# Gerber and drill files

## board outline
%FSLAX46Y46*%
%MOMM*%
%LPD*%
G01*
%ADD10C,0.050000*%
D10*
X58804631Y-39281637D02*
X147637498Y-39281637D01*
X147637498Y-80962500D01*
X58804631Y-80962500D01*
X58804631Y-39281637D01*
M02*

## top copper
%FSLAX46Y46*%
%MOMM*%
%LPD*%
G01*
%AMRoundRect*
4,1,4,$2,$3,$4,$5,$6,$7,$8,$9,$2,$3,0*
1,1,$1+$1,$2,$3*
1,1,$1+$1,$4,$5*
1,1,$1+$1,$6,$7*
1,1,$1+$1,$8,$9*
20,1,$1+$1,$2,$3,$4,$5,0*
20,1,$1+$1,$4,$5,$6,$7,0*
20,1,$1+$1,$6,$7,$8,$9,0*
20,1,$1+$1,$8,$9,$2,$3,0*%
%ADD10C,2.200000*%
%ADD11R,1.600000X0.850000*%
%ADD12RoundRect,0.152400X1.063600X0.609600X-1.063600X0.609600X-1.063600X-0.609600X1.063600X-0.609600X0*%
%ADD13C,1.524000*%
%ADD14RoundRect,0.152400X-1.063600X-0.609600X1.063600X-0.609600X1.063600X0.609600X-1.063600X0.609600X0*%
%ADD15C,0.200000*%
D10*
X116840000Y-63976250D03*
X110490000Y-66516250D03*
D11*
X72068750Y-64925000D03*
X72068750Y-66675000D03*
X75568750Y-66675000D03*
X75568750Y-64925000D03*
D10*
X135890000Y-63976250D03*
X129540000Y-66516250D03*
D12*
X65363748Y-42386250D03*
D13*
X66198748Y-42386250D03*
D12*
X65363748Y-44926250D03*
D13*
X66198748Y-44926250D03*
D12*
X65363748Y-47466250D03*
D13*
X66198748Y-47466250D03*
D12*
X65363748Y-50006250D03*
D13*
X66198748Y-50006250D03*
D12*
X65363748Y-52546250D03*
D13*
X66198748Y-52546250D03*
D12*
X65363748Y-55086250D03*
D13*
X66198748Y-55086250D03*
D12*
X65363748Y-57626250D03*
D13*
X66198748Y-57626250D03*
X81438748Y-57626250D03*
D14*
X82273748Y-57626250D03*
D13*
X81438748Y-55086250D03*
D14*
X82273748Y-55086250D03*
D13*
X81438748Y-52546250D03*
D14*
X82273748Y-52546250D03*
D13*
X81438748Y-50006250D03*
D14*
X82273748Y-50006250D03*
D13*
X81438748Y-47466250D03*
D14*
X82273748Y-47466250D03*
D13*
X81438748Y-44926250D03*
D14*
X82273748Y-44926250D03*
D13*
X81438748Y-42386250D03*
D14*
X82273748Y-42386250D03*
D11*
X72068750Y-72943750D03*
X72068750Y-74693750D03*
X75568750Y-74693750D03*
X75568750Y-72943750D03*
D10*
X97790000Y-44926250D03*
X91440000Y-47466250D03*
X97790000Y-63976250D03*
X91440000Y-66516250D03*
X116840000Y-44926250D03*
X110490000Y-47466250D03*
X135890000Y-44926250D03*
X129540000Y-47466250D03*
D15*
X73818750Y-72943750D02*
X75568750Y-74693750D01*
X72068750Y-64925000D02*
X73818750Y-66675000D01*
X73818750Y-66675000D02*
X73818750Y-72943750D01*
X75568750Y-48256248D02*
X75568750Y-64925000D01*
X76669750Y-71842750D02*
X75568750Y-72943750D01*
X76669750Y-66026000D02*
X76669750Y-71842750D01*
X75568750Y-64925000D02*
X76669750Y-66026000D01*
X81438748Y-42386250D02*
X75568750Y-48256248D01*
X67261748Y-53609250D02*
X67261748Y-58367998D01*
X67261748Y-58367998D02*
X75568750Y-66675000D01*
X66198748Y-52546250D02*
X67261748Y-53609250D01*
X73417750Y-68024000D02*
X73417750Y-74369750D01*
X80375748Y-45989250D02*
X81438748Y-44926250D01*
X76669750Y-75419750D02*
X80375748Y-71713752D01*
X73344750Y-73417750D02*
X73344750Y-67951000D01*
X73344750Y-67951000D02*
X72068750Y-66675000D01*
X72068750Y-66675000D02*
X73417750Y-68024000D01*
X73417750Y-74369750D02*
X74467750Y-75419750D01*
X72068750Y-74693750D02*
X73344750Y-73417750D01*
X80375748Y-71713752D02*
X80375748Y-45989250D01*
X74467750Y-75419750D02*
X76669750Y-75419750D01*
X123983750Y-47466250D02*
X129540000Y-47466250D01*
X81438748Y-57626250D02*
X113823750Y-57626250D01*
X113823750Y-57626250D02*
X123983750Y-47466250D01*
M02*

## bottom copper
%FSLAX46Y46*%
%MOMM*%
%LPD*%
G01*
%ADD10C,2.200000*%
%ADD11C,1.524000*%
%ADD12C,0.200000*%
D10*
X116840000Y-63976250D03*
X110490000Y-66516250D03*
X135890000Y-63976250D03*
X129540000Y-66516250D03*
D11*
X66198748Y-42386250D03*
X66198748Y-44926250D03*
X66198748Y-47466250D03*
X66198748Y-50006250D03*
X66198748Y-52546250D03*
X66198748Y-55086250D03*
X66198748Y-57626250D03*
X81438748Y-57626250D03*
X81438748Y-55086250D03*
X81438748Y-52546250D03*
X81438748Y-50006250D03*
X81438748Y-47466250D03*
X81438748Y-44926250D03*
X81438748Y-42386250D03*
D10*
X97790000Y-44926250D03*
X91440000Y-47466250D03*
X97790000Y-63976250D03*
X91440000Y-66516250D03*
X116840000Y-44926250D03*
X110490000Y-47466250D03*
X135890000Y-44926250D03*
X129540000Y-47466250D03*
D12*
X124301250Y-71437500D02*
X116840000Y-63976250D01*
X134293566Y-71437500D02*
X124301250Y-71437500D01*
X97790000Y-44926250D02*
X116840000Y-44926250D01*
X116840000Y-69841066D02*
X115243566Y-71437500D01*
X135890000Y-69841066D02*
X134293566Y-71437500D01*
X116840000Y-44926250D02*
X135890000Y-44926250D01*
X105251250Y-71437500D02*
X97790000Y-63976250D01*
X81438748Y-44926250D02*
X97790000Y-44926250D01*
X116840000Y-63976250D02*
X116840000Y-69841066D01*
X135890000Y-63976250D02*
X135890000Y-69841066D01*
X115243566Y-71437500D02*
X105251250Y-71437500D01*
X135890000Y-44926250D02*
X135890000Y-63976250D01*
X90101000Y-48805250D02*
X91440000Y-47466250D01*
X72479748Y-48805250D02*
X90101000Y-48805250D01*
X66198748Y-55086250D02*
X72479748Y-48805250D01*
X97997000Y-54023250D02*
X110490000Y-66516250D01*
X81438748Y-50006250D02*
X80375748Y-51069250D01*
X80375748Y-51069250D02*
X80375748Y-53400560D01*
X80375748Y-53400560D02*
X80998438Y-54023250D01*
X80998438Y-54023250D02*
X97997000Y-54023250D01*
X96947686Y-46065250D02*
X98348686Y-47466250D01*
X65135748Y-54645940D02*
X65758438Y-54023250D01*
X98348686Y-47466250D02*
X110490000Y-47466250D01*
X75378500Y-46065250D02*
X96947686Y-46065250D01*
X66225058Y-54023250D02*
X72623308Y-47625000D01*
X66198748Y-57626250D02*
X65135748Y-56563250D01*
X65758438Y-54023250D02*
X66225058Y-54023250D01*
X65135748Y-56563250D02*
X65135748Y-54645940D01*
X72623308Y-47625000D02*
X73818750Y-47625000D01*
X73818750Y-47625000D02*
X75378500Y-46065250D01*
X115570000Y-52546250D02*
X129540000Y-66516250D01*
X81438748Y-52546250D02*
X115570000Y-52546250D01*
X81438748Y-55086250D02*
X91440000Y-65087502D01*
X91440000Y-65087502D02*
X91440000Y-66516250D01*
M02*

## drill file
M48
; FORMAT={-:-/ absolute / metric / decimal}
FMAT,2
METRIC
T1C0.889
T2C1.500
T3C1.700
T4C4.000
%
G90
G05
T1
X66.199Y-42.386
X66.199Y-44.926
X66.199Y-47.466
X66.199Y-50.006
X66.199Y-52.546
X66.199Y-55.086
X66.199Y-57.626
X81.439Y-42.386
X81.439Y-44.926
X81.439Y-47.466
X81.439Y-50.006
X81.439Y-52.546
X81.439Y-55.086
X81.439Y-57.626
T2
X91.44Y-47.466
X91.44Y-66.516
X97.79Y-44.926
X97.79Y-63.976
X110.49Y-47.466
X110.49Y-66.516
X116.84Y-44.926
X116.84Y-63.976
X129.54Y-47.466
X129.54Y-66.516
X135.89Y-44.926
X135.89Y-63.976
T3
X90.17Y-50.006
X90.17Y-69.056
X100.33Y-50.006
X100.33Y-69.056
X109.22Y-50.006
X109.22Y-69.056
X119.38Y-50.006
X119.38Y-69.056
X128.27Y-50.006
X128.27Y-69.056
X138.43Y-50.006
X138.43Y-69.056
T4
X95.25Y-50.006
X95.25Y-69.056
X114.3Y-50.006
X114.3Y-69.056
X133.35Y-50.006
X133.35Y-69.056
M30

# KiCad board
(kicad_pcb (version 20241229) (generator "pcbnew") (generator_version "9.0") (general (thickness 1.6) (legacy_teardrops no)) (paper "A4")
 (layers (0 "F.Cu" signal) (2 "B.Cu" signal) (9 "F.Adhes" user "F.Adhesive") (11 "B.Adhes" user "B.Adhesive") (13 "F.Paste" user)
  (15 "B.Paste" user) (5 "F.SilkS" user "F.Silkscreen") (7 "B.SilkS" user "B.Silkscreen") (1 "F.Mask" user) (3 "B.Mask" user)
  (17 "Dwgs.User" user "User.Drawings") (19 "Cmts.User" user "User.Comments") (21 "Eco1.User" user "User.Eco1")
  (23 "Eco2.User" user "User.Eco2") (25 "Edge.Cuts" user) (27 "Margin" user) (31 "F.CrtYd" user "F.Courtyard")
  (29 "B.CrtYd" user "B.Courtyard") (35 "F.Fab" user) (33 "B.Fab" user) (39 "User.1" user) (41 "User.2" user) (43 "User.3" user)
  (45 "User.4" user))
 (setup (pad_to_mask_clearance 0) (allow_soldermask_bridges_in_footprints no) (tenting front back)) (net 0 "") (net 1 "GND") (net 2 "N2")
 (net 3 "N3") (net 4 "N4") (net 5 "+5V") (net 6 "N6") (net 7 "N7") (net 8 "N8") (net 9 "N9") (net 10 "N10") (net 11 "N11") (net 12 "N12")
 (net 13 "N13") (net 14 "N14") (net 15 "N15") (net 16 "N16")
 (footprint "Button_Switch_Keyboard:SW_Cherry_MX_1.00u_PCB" (layer "F.Cu") (at 116.84 63.97625)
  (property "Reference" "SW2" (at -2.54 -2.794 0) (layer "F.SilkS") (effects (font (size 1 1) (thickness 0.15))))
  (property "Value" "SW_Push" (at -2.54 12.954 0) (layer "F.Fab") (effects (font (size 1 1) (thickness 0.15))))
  (pad "" np_thru_hole circle (at -7.62 5.08) (size 1.7 1.7) (drill 1.7) (layers "*.Cu" "*.Mask"))
  (pad "" np_thru_hole circle (at -2.54 5.08) (size 4 4) (drill 4) (layers "*.Cu" "*.Mask"))
  (pad "" np_thru_hole circle (at 2.54 5.08) (size 1.7 1.7) (drill 1.7) (layers "*.Cu" "*.Mask"))
  (pad "1" thru_hole circle (at 0 0) (size 2.2 2.2) (drill 1.5) (layers "*.Cu" "*.Mask") (remove_unused_layers no) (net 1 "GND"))
  (pad "2" thru_hole circle (at -6.35 2.54) (size 2.2 2.2) (drill 1.5) (layers "*.Cu" "*.Mask") (remove_unused_layers no) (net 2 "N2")))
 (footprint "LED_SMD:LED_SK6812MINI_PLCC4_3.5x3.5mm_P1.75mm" (layer "F.Cu") (at 73.81875 65.8)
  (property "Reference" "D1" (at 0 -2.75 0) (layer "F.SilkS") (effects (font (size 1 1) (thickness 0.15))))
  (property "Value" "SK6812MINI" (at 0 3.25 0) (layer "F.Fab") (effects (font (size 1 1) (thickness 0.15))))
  (pad "1" smd rect (at -1.75 -0.875) (size 1.6 0.85) (layers "F.Cu" "F.Mask" "F.Paste") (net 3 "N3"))
  (pad "2" smd rect (at -1.75 0.875) (size 1.6 0.85) (layers "F.Cu" "F.Mask" "F.Paste") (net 1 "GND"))
  (pad "3" smd rect (at 1.75 0.875) (size 1.6 0.85) (layers "F.Cu" "F.Mask" "F.Paste") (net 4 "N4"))
  (pad "4" smd rect (at 1.75 -0.875) (size 1.6 0.85) (layers "F.Cu" "F.Mask" "F.Paste") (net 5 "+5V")))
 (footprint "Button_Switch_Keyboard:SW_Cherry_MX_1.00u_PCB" (layer "F.Cu") (at 135.89 63.97625)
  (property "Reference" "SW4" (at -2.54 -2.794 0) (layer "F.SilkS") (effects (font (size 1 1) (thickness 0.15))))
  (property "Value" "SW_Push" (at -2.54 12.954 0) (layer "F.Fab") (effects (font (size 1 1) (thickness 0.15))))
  (pad "" np_thru_hole circle (at -7.62 5.08) (size 1.7 1.7) (drill 1.7) (layers "*.Cu" "*.Mask"))
  (pad "" np_thru_hole circle (at -2.54 5.08) (size 4 4) (drill 4) (layers "*.Cu" "*.Mask"))
  (pad "" np_thru_hole circle (at 2.54 5.08) (size 1.7 1.7) (drill 1.7) (layers "*.Cu" "*.Mask"))
  (pad "1" thru_hole circle (at 0 0) (size 2.2 2.2) (drill 1.5) (layers "*.Cu" "*.Mask") (remove_unused_layers no) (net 1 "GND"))
  (pad "2" thru_hole circle (at -6.35 2.54) (size 2.2 2.2) (drill 1.5) (layers "*.Cu" "*.Mask") (remove_unused_layers no) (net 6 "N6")))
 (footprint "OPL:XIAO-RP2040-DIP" (layer "F.Cu") (at 73.818748 50.00625)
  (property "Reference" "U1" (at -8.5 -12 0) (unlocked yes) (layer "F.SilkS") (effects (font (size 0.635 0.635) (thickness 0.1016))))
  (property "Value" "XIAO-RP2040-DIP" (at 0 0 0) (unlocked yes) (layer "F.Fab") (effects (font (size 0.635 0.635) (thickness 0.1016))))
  (pad "1" smd roundrect (at -8.455 -7.62 180) (size 2.432 1.524) (layers "F.Cu" "F.Mask") (roundrect_rratio 0.1) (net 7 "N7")
   (thermal_bridge_angle 45))
  (pad "1" thru_hole circle (at -7.62 -7.62 180) (size 1.524 1.524) (drill 0.889) (layers "*.Cu" "*.Mask") (remove_unused_layers no)
   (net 7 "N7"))
  (pad "2" smd roundrect (at -8.455 -5.08 180) (size 2.432 1.524) (layers "F.Cu" "F.Mask") (roundrect_rratio 0.1) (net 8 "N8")
   (thermal_bridge_angle 45))
  (pad "2" thru_hole circle (at -7.62 -5.08 180) (size 1.524 1.524) (drill 0.889) (layers "*.Cu" "*.Mask") (remove_unused_layers no)
   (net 8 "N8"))
  (pad "3" smd roundrect (at -8.455 -2.54 180) (size 2.432 1.524) (layers "F.Cu" "F.Mask") (roundrect_rratio 0.1) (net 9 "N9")
   (thermal_bridge_angle 45))
  (pad "3" thru_hole circle (at -7.62 -2.54 180) (size 1.524 1.524) (drill 0.889) (layers "*.Cu" "*.Mask") (remove_unused_layers no)
   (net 9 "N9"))
  (pad "4" smd roundrect (at -8.455 0 180) (size 2.432 1.524) (layers "F.Cu" "F.Mask") (roundrect_rratio 0.1) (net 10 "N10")
   (thermal_bridge_angle 45))
  (pad "4" thru_hole circle (at -7.62 0 180) (size 1.524 1.524) (drill 0.889) (layers "*.Cu" "*.Mask") (remove_unused_layers no)
   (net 10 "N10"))
  (pad "5" smd roundrect (at -8.455 2.54 180) (size 2.432 1.524) (layers "F.Cu" "F.Mask") (roundrect_rratio 0.1) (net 4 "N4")
   (thermal_bridge_angle 45))
  (pad "5" thru_hole circle (at -7.62 2.54 180) (size 1.524 1.524) (drill 0.889) (layers "*.Cu" "*.Mask") (remove_unused_layers no)
   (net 4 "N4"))
  (pad "6" smd roundrect (at -8.455 5.08 180) (size 2.432 1.524) (layers "F.Cu" "F.Mask") (roundrect_rratio 0.1) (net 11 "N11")
   (thermal_bridge_angle 45))
  (pad "6" thru_hole circle (at -7.62 5.08 180) (size 1.524 1.524) (drill 0.889) (layers "*.Cu" "*.Mask") (remove_unused_layers no)
   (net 11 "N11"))
  (pad "7" smd roundrect (at -8.455 7.62 180) (size 2.432 1.524) (layers "F.Cu" "F.Mask") (roundrect_rratio 0.1) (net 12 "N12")
   (thermal_bridge_angle 45))
  (pad "7" thru_hole circle (at -7.62 7.62 180) (size 1.524 1.524) (drill 0.889) (layers "*.Cu" "*.Mask") (remove_unused_layers no)
   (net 12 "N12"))
  (pad "8" thru_hole circle (at 7.62 7.62) (size 1.524 1.524) (drill 0.889) (layers "*.Cu" "*.Mask") (remove_unused_layers no)
   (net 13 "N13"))
  (pad "8" smd roundrect (at 8.455 7.62) (size 2.432 1.524) (layers "F.Cu" "F.Mask") (roundrect_rratio 0.1) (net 13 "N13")
   (thermal_bridge_angle 45))
  (pad "9" thru_hole circle (at 7.62 5.08) (size 1.524 1.524) (drill 0.889) (layers "*.Cu" "*.Mask") (remove_unused_layers no)
   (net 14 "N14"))
  (pad "9" smd roundrect (at 8.455 5.08) (size 2.432 1.524) (layers "F.Cu" "F.Mask") (roundrect_rratio 0.1) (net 14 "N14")
   (thermal_bridge_angle 45))
  (pad "10" thru_hole circle (at 7.62 2.54) (size 1.524 1.524) (drill 0.889) (layers "*.Cu" "*.Mask") (remove_unused_layers no) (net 6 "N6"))
  (pad "10" smd roundrect (at 8.455 2.54) (size 2.432 1.524) (layers "F.Cu" "F.Mask") (roundrect_rratio 0.1) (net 6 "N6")
   (thermal_bridge_angle 45))
  (pad "11" thru_hole circle (at 7.62 0) (size 1.524 1.524) (drill 0.889) (layers "*.Cu" "*.Mask") (remove_unused_layers no) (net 2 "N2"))
  (pad "11" smd roundrect (at 8.455 0) (size 2.432 1.524) (layers "F.Cu" "F.Mask") (roundrect_rratio 0.1) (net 2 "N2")
   (thermal_bridge_angle 45))
  (pad "12" thru_hole circle (at 7.62 -2.54) (size 1.524 1.524) (drill 0.889) (layers "*.Cu" "*.Mask") (remove_unused_layers no)
   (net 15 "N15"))
  (pad "12" smd roundrect (at 8.455 -2.54) (size 2.432 1.524) (layers "F.Cu" "F.Mask") (roundrect_rratio 0.1) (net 15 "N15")
   (thermal_bridge_angle 45))
  (pad "13" thru_hole circle (at 7.62 -5.08) (size 1.524 1.524) (drill 0.889) (layers "*.Cu" "*.Mask") (remove_unused_layers no)
   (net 1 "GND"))
  (pad "13" smd roundrect (at 8.455 -5.08) (size 2.432 1.524) (layers "F.Cu" "F.Mask") (roundrect_rratio 0.1) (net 1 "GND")
   (thermal_bridge_angle 45))
  (pad "14" thru_hole circle (at 7.62 -7.62) (size 1.524 1.524) (drill 0.889) (layers "*.Cu" "*.Mask") (remove_unused_layers no)
   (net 5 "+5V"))
  (pad "14" smd roundrect (at 8.455 -7.62) (size 2.432 1.524) (layers "F.Cu" "F.Mask") (roundrect_rratio 0.1) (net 5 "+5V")
   (thermal_bridge_angle 45)))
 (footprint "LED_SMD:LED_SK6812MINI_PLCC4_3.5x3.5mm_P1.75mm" (layer "F.Cu") (at 73.81875 73.81875)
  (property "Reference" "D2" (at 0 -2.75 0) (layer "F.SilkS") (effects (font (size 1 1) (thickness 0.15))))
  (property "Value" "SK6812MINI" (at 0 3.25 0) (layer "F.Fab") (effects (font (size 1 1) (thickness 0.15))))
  (pad "1" smd rect (at -1.75 -0.875) (size 1.6 0.85) (layers "F.Cu" "F.Mask" "F.Paste") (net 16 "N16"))
  (pad "2" smd rect (at -1.75 0.875) (size 1.6 0.85) (layers "F.Cu" "F.Mask" "F.Paste") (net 1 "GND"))
  (pad "3" smd rect (at 1.75 0.875) (size 1.6 0.85) (layers "F.Cu" "F.Mask" "F.Paste") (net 3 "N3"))
  (pad "4" smd rect (at 1.75 -0.875) (size 1.6 0.85) (layers "F.Cu" "F.Mask" "F.Paste") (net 5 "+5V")))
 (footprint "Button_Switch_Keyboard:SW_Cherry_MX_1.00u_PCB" (layer "F.Cu") (at 97.79 44.92625)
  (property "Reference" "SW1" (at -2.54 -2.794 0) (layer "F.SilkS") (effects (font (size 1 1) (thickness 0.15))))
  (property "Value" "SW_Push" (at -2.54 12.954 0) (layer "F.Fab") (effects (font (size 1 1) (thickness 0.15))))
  (pad "" np_thru_hole circle (at -7.62 5.08) (size 1.7 1.7) (drill 1.7) (layers "*.Cu" "*.Mask"))
  (pad "" np_thru_hole circle (at -2.54 5.08) (size 4 4) (drill 4) (layers "*.Cu" "*.Mask"))
  (pad "" np_thru_hole circle (at 2.54 5.08) (size 1.7 1.7) (drill 1.7) (layers "*.Cu" "*.Mask"))
  (pad "1" thru_hole circle (at 0 0) (size 2.2 2.2) (drill 1.5) (layers "*.Cu" "*.Mask") (remove_unused_layers no) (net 1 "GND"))
  (pad "2" thru_hole circle (at -6.35 2.54) (size 2.2 2.2) (drill 1.5) (layers "*.Cu" "*.Mask") (remove_unused_layers no) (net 11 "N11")))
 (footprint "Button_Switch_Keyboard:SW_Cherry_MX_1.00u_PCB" (layer "F.Cu") (at 97.79 63.97625)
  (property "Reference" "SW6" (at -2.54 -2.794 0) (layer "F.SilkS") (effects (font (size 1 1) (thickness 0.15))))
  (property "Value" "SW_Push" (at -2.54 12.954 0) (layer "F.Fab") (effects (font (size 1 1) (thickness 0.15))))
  (pad "" np_thru_hole circle (at -7.62 5.08) (size 1.7 1.7) (drill 1.7) (layers "*.Cu" "*.Mask"))
  (pad "" np_thru_hole circle (at -2.54 5.08) (size 4 4) (drill 4) (layers "*.Cu" "*.Mask"))
  (pad "" np_thru_hole circle (at 2.54 5.08) (size 1.7 1.7) (drill 1.7) (layers "*.Cu" "*.Mask"))
  (pad "1" thru_hole circle (at 0 0) (size 2.2 2.2) (drill 1.5) (layers "*.Cu" "*.Mask") (remove_unused_layers no) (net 1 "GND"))
  (pad "2" thru_hole circle (at -6.35 2.54) (size 2.2 2.2) (drill 1.5) (layers "*.Cu" "*.Mask") (remove_unused_layers no) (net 14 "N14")))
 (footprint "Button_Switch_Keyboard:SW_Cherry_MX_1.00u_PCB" (layer "F.Cu") (at 116.84 44.92625)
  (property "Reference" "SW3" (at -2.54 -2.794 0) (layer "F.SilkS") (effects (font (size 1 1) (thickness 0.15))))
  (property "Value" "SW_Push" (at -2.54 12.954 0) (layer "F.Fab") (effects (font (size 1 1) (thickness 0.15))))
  (pad "" np_thru_hole circle (at -7.62 5.08) (size 1.7 1.7) (drill 1.7) (layers "*.Cu" "*.Mask"))
  (pad "" np_thru_hole circle (at -2.54 5.08) (size 4 4) (drill 4) (layers "*.Cu" "*.Mask"))
  (pad "" np_thru_hole circle (at 2.54 5.08) (size 1.7 1.7) (drill 1.7) (layers "*.Cu" "*.Mask"))
  (pad "1" thru_hole circle (at 0 0) (size 2.2 2.2) (drill 1.5) (layers "*.Cu" "*.Mask") (remove_unused_layers no) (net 1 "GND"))
  (pad "2" thru_hole circle (at -6.35 2.54) (size 2.2 2.2) (drill 1.5) (layers "*.Cu" "*.Mask") (remove_unused_layers no) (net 12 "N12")))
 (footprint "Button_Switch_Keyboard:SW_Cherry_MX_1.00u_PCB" (layer "F.Cu") (at 135.89 44.92625)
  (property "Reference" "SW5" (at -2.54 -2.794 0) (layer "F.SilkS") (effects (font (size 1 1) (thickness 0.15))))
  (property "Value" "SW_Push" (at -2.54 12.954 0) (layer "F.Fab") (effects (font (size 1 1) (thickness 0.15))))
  (pad "" np_thru_hole circle (at -7.62 5.08) (size 1.7 1.7) (drill 1.7) (layers "*.Cu" "*.Mask"))
  (pad "" np_thru_hole circle (at -2.54 5.08) (size 4 4) (drill 4) (layers "*.Cu" "*.Mask"))
  (pad "" np_thru_hole circle (at 2.54 5.08) (size 1.7 1.7) (drill 1.7) (layers "*.Cu" "*.Mask"))
  (pad "1" thru_hole circle (at 0 0) (size 2.2 2.2) (drill 1.5) (layers "*.Cu" "*.Mask") (remove_unused_layers no) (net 1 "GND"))
  (pad "2" thru_hole circle (at -6.35 2.54) (size 2.2 2.2) (drill 1.5) (layers "*.Cu" "*.Mask") (remove_unused_layers no) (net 13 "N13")))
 (gr_rect (start 58.804631 39.281637) (end 147.637498 80.9625) (stroke (width 0.05) (type default)) (fill no) (layer "Edge.Cuts"))
 (segment (start 73.81875 72.94375) (end 75.56875 74.69375) (width 0.2) (layer "F.Cu") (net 3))
 (segment (start 72.06875 64.925) (end 73.81875 66.675) (width 0.2) (layer "F.Cu") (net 3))
 (segment (start 73.81875 66.675) (end 73.81875 72.94375) (width 0.2) (layer "F.Cu") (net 3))
 (segment (start 75.56875 48.256248) (end 75.56875 64.925) (width 0.2) (layer "F.Cu") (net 5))
 (segment (start 76.66975 71.84275) (end 75.56875 72.94375) (width 0.2) (layer "F.Cu") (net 5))
 (segment (start 76.66975 66.026) (end 76.66975 71.84275) (width 0.2) (layer "F.Cu") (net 5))
 (segment (start 75.56875 64.925) (end 76.66975 66.026) (width 0.2) (layer "F.Cu") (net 5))
 (segment (start 81.438748 42.38625) (end 75.56875 48.256248) (width 0.2) (layer "F.Cu") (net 5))
 (segment (start 67.261748 53.60925) (end 67.261748 58.367998) (width 0.2) (layer "F.Cu") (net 4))
 (segment (start 67.261748 58.367998) (end 75.56875 66.675) (width 0.2) (layer "F.Cu") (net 4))
 (segment (start 66.198748 52.54625) (end 67.261748 53.60925) (width 0.2) (layer "F.Cu") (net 4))
 (segment (start 73.41775 68.024) (end 73.41775 74.36975) (width 0.2) (layer "F.Cu") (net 1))
 (segment (start 80.375748 45.98925) (end 81.438748 44.92625) (width 0.2) (layer "F.Cu") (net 1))
 (segment (start 76.66975 75.41975) (end 80.375748 71.713752) (width 0.2) (layer "F.Cu") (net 1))
 (segment (start 73.34475 73.41775) (end 73.34475 67.951) (width 0.2) (layer "F.Cu") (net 1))
 (segment (start 73.34475 67.951) (end 72.06875 66.675) (width 0.2) (layer "F.Cu") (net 1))
 (segment (start 72.06875 66.675) (end 73.41775 68.024) (width 0.2) (layer "F.Cu") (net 1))
 (segment (start 73.41775 74.36975) (end 74.46775 75.41975) (width 0.2) (layer "F.Cu") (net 1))
 (segment (start 72.06875 74.69375) (end 73.34475 73.41775) (width 0.2) (layer "F.Cu") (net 1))
 (segment (start 80.375748 71.713752) (end 80.375748 45.98925) (width 0.2) (layer "F.Cu") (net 1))
 (segment (start 74.46775 75.41975) (end 76.66975 75.41975) (width 0.2) (layer "F.Cu") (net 1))
 (segment (start 124.30125 71.4375) (end 116.84 63.97625) (width 0.2) (layer "B.Cu") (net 1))
 (segment (start 134.293566 71.4375) (end 124.30125 71.4375) (width 0.2) (layer "B.Cu") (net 1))
 (segment (start 97.79 44.92625) (end 116.84 44.92625) (width 0.2) (layer "B.Cu") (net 1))
 (segment (start 116.84 69.841066) (end 115.243566 71.4375) (width 0.2) (layer "B.Cu") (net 1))
 (segment (start 135.89 69.841066) (end 134.293566 71.4375) (width 0.2) (layer "B.Cu") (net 1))
 (segment (start 116.84 44.92625) (end 135.89 44.92625) (width 0.2) (layer "B.Cu") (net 1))
 (segment (start 105.25125 71.4375) (end 97.79 63.97625) (width 0.2) (layer "B.Cu") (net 1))
 (segment (start 81.438748 44.92625) (end 97.79 44.92625) (width 0.2) (layer "B.Cu") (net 1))
 (segment (start 116.84 63.97625) (end 116.84 69.841066) (width 0.2) (layer "B.Cu") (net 1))
 (segment (start 135.89 63.97625) (end 135.89 69.841066) (width 0.2) (layer "B.Cu") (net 1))
 (segment (start 115.243566 71.4375) (end 105.25125 71.4375) (width 0.2) (layer "B.Cu") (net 1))
 (segment (start 135.89 44.92625) (end 135.89 63.97625) (width 0.2) (layer "B.Cu") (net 1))
 (segment (start 90.101 48.80525) (end 91.44 47.46625) (width 0.2) (layer "B.Cu") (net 11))
 (segment (start 72.479748 48.80525) (end 90.101 48.80525) (width 0.2) (layer "B.Cu") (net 11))
 (segment (start 66.198748 55.08625) (end 72.479748 48.80525) (width 0.2) (layer "B.Cu") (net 11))
 (segment (start 97.997 54.02325) (end 110.49 66.51625) (width 0.2) (layer "B.Cu") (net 2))
 (segment (start 81.438748 50.00625) (end 80.375748 51.06925) (width 0.2) (layer "B.Cu") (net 2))
 (segment (start 80.375748 51.06925) (end 80.375748 53.40056) (width 0.2) (layer "B.Cu") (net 2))
 (segment (start 80.375748 53.40056) (end 80.998438 54.02325) (width 0.2) (layer "B.Cu") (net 2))
 (segment (start 80.998438 54.02325) (end 97.997 54.02325) (width 0.2) (layer "B.Cu") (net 2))
 (segment (start 96.947686 46.06525) (end 98.348686 47.46625) (width 0.2) (layer "B.Cu") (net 12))
 (segment (start 65.135748 54.64594) (end 65.758438 54.02325) (width 0.2) (layer "B.Cu") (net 12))
 (segment (start 98.348686 47.46625) (end 110.49 47.46625) (width 0.2) (layer "B.Cu") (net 12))
 (segment (start 75.3785 46.06525) (end 96.947686 46.06525) (width 0.2) (layer "B.Cu") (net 12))
 (segment (start 66.225058 54.02325) (end 72.623308 47.625) (width 0.2) (layer "B.Cu") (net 12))
 (segment (start 66.198748 57.62625) (end 65.135748 56.56325) (width 0.2) (layer "B.Cu") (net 12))
 (segment (start 65.758438 54.02325) (end 66.225058 54.02325) (width 0.2) (layer "B.Cu") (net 12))
 (segment (start 65.135748 56.56325) (end 65.135748 54.64594) (width 0.2) (layer "B.Cu") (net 12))
 (segment (start 72.623308 47.625) (end 73.81875 47.625) (width 0.2) (layer "B.Cu") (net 12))
 (segment (start 73.81875 47.625) (end 75.3785 46.06525) (width 0.2) (layer "B.Cu") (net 12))
 (segment (start 115.57 52.54625) (end 129.54 66.51625) (width 0.2) (layer "B.Cu") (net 6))
 (segment (start 81.438748 52.54625) (end 115.57 52.54625) (width 0.2) (layer "B.Cu") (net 6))
 (segment (start 123.98375 47.46625) (end 129.54 47.46625) (width 0.2) (layer "F.Cu") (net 13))
 (segment (start 81.438748 57.62625) (end 113.82375 57.62625) (width 0.2) (layer "F.Cu") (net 13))
 (segment (start 113.82375 57.62625) (end 123.98375 47.46625) (width 0.2) (layer "F.Cu") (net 13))
 (segment (start 81.438748 55.08625) (end 91.44 65.087502) (width 0.2) (layer "B.Cu") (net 14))
 (segment (start 91.44 65.087502) (end 91.44 66.51625) (width 0.2) (layer "B.Cu") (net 14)))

